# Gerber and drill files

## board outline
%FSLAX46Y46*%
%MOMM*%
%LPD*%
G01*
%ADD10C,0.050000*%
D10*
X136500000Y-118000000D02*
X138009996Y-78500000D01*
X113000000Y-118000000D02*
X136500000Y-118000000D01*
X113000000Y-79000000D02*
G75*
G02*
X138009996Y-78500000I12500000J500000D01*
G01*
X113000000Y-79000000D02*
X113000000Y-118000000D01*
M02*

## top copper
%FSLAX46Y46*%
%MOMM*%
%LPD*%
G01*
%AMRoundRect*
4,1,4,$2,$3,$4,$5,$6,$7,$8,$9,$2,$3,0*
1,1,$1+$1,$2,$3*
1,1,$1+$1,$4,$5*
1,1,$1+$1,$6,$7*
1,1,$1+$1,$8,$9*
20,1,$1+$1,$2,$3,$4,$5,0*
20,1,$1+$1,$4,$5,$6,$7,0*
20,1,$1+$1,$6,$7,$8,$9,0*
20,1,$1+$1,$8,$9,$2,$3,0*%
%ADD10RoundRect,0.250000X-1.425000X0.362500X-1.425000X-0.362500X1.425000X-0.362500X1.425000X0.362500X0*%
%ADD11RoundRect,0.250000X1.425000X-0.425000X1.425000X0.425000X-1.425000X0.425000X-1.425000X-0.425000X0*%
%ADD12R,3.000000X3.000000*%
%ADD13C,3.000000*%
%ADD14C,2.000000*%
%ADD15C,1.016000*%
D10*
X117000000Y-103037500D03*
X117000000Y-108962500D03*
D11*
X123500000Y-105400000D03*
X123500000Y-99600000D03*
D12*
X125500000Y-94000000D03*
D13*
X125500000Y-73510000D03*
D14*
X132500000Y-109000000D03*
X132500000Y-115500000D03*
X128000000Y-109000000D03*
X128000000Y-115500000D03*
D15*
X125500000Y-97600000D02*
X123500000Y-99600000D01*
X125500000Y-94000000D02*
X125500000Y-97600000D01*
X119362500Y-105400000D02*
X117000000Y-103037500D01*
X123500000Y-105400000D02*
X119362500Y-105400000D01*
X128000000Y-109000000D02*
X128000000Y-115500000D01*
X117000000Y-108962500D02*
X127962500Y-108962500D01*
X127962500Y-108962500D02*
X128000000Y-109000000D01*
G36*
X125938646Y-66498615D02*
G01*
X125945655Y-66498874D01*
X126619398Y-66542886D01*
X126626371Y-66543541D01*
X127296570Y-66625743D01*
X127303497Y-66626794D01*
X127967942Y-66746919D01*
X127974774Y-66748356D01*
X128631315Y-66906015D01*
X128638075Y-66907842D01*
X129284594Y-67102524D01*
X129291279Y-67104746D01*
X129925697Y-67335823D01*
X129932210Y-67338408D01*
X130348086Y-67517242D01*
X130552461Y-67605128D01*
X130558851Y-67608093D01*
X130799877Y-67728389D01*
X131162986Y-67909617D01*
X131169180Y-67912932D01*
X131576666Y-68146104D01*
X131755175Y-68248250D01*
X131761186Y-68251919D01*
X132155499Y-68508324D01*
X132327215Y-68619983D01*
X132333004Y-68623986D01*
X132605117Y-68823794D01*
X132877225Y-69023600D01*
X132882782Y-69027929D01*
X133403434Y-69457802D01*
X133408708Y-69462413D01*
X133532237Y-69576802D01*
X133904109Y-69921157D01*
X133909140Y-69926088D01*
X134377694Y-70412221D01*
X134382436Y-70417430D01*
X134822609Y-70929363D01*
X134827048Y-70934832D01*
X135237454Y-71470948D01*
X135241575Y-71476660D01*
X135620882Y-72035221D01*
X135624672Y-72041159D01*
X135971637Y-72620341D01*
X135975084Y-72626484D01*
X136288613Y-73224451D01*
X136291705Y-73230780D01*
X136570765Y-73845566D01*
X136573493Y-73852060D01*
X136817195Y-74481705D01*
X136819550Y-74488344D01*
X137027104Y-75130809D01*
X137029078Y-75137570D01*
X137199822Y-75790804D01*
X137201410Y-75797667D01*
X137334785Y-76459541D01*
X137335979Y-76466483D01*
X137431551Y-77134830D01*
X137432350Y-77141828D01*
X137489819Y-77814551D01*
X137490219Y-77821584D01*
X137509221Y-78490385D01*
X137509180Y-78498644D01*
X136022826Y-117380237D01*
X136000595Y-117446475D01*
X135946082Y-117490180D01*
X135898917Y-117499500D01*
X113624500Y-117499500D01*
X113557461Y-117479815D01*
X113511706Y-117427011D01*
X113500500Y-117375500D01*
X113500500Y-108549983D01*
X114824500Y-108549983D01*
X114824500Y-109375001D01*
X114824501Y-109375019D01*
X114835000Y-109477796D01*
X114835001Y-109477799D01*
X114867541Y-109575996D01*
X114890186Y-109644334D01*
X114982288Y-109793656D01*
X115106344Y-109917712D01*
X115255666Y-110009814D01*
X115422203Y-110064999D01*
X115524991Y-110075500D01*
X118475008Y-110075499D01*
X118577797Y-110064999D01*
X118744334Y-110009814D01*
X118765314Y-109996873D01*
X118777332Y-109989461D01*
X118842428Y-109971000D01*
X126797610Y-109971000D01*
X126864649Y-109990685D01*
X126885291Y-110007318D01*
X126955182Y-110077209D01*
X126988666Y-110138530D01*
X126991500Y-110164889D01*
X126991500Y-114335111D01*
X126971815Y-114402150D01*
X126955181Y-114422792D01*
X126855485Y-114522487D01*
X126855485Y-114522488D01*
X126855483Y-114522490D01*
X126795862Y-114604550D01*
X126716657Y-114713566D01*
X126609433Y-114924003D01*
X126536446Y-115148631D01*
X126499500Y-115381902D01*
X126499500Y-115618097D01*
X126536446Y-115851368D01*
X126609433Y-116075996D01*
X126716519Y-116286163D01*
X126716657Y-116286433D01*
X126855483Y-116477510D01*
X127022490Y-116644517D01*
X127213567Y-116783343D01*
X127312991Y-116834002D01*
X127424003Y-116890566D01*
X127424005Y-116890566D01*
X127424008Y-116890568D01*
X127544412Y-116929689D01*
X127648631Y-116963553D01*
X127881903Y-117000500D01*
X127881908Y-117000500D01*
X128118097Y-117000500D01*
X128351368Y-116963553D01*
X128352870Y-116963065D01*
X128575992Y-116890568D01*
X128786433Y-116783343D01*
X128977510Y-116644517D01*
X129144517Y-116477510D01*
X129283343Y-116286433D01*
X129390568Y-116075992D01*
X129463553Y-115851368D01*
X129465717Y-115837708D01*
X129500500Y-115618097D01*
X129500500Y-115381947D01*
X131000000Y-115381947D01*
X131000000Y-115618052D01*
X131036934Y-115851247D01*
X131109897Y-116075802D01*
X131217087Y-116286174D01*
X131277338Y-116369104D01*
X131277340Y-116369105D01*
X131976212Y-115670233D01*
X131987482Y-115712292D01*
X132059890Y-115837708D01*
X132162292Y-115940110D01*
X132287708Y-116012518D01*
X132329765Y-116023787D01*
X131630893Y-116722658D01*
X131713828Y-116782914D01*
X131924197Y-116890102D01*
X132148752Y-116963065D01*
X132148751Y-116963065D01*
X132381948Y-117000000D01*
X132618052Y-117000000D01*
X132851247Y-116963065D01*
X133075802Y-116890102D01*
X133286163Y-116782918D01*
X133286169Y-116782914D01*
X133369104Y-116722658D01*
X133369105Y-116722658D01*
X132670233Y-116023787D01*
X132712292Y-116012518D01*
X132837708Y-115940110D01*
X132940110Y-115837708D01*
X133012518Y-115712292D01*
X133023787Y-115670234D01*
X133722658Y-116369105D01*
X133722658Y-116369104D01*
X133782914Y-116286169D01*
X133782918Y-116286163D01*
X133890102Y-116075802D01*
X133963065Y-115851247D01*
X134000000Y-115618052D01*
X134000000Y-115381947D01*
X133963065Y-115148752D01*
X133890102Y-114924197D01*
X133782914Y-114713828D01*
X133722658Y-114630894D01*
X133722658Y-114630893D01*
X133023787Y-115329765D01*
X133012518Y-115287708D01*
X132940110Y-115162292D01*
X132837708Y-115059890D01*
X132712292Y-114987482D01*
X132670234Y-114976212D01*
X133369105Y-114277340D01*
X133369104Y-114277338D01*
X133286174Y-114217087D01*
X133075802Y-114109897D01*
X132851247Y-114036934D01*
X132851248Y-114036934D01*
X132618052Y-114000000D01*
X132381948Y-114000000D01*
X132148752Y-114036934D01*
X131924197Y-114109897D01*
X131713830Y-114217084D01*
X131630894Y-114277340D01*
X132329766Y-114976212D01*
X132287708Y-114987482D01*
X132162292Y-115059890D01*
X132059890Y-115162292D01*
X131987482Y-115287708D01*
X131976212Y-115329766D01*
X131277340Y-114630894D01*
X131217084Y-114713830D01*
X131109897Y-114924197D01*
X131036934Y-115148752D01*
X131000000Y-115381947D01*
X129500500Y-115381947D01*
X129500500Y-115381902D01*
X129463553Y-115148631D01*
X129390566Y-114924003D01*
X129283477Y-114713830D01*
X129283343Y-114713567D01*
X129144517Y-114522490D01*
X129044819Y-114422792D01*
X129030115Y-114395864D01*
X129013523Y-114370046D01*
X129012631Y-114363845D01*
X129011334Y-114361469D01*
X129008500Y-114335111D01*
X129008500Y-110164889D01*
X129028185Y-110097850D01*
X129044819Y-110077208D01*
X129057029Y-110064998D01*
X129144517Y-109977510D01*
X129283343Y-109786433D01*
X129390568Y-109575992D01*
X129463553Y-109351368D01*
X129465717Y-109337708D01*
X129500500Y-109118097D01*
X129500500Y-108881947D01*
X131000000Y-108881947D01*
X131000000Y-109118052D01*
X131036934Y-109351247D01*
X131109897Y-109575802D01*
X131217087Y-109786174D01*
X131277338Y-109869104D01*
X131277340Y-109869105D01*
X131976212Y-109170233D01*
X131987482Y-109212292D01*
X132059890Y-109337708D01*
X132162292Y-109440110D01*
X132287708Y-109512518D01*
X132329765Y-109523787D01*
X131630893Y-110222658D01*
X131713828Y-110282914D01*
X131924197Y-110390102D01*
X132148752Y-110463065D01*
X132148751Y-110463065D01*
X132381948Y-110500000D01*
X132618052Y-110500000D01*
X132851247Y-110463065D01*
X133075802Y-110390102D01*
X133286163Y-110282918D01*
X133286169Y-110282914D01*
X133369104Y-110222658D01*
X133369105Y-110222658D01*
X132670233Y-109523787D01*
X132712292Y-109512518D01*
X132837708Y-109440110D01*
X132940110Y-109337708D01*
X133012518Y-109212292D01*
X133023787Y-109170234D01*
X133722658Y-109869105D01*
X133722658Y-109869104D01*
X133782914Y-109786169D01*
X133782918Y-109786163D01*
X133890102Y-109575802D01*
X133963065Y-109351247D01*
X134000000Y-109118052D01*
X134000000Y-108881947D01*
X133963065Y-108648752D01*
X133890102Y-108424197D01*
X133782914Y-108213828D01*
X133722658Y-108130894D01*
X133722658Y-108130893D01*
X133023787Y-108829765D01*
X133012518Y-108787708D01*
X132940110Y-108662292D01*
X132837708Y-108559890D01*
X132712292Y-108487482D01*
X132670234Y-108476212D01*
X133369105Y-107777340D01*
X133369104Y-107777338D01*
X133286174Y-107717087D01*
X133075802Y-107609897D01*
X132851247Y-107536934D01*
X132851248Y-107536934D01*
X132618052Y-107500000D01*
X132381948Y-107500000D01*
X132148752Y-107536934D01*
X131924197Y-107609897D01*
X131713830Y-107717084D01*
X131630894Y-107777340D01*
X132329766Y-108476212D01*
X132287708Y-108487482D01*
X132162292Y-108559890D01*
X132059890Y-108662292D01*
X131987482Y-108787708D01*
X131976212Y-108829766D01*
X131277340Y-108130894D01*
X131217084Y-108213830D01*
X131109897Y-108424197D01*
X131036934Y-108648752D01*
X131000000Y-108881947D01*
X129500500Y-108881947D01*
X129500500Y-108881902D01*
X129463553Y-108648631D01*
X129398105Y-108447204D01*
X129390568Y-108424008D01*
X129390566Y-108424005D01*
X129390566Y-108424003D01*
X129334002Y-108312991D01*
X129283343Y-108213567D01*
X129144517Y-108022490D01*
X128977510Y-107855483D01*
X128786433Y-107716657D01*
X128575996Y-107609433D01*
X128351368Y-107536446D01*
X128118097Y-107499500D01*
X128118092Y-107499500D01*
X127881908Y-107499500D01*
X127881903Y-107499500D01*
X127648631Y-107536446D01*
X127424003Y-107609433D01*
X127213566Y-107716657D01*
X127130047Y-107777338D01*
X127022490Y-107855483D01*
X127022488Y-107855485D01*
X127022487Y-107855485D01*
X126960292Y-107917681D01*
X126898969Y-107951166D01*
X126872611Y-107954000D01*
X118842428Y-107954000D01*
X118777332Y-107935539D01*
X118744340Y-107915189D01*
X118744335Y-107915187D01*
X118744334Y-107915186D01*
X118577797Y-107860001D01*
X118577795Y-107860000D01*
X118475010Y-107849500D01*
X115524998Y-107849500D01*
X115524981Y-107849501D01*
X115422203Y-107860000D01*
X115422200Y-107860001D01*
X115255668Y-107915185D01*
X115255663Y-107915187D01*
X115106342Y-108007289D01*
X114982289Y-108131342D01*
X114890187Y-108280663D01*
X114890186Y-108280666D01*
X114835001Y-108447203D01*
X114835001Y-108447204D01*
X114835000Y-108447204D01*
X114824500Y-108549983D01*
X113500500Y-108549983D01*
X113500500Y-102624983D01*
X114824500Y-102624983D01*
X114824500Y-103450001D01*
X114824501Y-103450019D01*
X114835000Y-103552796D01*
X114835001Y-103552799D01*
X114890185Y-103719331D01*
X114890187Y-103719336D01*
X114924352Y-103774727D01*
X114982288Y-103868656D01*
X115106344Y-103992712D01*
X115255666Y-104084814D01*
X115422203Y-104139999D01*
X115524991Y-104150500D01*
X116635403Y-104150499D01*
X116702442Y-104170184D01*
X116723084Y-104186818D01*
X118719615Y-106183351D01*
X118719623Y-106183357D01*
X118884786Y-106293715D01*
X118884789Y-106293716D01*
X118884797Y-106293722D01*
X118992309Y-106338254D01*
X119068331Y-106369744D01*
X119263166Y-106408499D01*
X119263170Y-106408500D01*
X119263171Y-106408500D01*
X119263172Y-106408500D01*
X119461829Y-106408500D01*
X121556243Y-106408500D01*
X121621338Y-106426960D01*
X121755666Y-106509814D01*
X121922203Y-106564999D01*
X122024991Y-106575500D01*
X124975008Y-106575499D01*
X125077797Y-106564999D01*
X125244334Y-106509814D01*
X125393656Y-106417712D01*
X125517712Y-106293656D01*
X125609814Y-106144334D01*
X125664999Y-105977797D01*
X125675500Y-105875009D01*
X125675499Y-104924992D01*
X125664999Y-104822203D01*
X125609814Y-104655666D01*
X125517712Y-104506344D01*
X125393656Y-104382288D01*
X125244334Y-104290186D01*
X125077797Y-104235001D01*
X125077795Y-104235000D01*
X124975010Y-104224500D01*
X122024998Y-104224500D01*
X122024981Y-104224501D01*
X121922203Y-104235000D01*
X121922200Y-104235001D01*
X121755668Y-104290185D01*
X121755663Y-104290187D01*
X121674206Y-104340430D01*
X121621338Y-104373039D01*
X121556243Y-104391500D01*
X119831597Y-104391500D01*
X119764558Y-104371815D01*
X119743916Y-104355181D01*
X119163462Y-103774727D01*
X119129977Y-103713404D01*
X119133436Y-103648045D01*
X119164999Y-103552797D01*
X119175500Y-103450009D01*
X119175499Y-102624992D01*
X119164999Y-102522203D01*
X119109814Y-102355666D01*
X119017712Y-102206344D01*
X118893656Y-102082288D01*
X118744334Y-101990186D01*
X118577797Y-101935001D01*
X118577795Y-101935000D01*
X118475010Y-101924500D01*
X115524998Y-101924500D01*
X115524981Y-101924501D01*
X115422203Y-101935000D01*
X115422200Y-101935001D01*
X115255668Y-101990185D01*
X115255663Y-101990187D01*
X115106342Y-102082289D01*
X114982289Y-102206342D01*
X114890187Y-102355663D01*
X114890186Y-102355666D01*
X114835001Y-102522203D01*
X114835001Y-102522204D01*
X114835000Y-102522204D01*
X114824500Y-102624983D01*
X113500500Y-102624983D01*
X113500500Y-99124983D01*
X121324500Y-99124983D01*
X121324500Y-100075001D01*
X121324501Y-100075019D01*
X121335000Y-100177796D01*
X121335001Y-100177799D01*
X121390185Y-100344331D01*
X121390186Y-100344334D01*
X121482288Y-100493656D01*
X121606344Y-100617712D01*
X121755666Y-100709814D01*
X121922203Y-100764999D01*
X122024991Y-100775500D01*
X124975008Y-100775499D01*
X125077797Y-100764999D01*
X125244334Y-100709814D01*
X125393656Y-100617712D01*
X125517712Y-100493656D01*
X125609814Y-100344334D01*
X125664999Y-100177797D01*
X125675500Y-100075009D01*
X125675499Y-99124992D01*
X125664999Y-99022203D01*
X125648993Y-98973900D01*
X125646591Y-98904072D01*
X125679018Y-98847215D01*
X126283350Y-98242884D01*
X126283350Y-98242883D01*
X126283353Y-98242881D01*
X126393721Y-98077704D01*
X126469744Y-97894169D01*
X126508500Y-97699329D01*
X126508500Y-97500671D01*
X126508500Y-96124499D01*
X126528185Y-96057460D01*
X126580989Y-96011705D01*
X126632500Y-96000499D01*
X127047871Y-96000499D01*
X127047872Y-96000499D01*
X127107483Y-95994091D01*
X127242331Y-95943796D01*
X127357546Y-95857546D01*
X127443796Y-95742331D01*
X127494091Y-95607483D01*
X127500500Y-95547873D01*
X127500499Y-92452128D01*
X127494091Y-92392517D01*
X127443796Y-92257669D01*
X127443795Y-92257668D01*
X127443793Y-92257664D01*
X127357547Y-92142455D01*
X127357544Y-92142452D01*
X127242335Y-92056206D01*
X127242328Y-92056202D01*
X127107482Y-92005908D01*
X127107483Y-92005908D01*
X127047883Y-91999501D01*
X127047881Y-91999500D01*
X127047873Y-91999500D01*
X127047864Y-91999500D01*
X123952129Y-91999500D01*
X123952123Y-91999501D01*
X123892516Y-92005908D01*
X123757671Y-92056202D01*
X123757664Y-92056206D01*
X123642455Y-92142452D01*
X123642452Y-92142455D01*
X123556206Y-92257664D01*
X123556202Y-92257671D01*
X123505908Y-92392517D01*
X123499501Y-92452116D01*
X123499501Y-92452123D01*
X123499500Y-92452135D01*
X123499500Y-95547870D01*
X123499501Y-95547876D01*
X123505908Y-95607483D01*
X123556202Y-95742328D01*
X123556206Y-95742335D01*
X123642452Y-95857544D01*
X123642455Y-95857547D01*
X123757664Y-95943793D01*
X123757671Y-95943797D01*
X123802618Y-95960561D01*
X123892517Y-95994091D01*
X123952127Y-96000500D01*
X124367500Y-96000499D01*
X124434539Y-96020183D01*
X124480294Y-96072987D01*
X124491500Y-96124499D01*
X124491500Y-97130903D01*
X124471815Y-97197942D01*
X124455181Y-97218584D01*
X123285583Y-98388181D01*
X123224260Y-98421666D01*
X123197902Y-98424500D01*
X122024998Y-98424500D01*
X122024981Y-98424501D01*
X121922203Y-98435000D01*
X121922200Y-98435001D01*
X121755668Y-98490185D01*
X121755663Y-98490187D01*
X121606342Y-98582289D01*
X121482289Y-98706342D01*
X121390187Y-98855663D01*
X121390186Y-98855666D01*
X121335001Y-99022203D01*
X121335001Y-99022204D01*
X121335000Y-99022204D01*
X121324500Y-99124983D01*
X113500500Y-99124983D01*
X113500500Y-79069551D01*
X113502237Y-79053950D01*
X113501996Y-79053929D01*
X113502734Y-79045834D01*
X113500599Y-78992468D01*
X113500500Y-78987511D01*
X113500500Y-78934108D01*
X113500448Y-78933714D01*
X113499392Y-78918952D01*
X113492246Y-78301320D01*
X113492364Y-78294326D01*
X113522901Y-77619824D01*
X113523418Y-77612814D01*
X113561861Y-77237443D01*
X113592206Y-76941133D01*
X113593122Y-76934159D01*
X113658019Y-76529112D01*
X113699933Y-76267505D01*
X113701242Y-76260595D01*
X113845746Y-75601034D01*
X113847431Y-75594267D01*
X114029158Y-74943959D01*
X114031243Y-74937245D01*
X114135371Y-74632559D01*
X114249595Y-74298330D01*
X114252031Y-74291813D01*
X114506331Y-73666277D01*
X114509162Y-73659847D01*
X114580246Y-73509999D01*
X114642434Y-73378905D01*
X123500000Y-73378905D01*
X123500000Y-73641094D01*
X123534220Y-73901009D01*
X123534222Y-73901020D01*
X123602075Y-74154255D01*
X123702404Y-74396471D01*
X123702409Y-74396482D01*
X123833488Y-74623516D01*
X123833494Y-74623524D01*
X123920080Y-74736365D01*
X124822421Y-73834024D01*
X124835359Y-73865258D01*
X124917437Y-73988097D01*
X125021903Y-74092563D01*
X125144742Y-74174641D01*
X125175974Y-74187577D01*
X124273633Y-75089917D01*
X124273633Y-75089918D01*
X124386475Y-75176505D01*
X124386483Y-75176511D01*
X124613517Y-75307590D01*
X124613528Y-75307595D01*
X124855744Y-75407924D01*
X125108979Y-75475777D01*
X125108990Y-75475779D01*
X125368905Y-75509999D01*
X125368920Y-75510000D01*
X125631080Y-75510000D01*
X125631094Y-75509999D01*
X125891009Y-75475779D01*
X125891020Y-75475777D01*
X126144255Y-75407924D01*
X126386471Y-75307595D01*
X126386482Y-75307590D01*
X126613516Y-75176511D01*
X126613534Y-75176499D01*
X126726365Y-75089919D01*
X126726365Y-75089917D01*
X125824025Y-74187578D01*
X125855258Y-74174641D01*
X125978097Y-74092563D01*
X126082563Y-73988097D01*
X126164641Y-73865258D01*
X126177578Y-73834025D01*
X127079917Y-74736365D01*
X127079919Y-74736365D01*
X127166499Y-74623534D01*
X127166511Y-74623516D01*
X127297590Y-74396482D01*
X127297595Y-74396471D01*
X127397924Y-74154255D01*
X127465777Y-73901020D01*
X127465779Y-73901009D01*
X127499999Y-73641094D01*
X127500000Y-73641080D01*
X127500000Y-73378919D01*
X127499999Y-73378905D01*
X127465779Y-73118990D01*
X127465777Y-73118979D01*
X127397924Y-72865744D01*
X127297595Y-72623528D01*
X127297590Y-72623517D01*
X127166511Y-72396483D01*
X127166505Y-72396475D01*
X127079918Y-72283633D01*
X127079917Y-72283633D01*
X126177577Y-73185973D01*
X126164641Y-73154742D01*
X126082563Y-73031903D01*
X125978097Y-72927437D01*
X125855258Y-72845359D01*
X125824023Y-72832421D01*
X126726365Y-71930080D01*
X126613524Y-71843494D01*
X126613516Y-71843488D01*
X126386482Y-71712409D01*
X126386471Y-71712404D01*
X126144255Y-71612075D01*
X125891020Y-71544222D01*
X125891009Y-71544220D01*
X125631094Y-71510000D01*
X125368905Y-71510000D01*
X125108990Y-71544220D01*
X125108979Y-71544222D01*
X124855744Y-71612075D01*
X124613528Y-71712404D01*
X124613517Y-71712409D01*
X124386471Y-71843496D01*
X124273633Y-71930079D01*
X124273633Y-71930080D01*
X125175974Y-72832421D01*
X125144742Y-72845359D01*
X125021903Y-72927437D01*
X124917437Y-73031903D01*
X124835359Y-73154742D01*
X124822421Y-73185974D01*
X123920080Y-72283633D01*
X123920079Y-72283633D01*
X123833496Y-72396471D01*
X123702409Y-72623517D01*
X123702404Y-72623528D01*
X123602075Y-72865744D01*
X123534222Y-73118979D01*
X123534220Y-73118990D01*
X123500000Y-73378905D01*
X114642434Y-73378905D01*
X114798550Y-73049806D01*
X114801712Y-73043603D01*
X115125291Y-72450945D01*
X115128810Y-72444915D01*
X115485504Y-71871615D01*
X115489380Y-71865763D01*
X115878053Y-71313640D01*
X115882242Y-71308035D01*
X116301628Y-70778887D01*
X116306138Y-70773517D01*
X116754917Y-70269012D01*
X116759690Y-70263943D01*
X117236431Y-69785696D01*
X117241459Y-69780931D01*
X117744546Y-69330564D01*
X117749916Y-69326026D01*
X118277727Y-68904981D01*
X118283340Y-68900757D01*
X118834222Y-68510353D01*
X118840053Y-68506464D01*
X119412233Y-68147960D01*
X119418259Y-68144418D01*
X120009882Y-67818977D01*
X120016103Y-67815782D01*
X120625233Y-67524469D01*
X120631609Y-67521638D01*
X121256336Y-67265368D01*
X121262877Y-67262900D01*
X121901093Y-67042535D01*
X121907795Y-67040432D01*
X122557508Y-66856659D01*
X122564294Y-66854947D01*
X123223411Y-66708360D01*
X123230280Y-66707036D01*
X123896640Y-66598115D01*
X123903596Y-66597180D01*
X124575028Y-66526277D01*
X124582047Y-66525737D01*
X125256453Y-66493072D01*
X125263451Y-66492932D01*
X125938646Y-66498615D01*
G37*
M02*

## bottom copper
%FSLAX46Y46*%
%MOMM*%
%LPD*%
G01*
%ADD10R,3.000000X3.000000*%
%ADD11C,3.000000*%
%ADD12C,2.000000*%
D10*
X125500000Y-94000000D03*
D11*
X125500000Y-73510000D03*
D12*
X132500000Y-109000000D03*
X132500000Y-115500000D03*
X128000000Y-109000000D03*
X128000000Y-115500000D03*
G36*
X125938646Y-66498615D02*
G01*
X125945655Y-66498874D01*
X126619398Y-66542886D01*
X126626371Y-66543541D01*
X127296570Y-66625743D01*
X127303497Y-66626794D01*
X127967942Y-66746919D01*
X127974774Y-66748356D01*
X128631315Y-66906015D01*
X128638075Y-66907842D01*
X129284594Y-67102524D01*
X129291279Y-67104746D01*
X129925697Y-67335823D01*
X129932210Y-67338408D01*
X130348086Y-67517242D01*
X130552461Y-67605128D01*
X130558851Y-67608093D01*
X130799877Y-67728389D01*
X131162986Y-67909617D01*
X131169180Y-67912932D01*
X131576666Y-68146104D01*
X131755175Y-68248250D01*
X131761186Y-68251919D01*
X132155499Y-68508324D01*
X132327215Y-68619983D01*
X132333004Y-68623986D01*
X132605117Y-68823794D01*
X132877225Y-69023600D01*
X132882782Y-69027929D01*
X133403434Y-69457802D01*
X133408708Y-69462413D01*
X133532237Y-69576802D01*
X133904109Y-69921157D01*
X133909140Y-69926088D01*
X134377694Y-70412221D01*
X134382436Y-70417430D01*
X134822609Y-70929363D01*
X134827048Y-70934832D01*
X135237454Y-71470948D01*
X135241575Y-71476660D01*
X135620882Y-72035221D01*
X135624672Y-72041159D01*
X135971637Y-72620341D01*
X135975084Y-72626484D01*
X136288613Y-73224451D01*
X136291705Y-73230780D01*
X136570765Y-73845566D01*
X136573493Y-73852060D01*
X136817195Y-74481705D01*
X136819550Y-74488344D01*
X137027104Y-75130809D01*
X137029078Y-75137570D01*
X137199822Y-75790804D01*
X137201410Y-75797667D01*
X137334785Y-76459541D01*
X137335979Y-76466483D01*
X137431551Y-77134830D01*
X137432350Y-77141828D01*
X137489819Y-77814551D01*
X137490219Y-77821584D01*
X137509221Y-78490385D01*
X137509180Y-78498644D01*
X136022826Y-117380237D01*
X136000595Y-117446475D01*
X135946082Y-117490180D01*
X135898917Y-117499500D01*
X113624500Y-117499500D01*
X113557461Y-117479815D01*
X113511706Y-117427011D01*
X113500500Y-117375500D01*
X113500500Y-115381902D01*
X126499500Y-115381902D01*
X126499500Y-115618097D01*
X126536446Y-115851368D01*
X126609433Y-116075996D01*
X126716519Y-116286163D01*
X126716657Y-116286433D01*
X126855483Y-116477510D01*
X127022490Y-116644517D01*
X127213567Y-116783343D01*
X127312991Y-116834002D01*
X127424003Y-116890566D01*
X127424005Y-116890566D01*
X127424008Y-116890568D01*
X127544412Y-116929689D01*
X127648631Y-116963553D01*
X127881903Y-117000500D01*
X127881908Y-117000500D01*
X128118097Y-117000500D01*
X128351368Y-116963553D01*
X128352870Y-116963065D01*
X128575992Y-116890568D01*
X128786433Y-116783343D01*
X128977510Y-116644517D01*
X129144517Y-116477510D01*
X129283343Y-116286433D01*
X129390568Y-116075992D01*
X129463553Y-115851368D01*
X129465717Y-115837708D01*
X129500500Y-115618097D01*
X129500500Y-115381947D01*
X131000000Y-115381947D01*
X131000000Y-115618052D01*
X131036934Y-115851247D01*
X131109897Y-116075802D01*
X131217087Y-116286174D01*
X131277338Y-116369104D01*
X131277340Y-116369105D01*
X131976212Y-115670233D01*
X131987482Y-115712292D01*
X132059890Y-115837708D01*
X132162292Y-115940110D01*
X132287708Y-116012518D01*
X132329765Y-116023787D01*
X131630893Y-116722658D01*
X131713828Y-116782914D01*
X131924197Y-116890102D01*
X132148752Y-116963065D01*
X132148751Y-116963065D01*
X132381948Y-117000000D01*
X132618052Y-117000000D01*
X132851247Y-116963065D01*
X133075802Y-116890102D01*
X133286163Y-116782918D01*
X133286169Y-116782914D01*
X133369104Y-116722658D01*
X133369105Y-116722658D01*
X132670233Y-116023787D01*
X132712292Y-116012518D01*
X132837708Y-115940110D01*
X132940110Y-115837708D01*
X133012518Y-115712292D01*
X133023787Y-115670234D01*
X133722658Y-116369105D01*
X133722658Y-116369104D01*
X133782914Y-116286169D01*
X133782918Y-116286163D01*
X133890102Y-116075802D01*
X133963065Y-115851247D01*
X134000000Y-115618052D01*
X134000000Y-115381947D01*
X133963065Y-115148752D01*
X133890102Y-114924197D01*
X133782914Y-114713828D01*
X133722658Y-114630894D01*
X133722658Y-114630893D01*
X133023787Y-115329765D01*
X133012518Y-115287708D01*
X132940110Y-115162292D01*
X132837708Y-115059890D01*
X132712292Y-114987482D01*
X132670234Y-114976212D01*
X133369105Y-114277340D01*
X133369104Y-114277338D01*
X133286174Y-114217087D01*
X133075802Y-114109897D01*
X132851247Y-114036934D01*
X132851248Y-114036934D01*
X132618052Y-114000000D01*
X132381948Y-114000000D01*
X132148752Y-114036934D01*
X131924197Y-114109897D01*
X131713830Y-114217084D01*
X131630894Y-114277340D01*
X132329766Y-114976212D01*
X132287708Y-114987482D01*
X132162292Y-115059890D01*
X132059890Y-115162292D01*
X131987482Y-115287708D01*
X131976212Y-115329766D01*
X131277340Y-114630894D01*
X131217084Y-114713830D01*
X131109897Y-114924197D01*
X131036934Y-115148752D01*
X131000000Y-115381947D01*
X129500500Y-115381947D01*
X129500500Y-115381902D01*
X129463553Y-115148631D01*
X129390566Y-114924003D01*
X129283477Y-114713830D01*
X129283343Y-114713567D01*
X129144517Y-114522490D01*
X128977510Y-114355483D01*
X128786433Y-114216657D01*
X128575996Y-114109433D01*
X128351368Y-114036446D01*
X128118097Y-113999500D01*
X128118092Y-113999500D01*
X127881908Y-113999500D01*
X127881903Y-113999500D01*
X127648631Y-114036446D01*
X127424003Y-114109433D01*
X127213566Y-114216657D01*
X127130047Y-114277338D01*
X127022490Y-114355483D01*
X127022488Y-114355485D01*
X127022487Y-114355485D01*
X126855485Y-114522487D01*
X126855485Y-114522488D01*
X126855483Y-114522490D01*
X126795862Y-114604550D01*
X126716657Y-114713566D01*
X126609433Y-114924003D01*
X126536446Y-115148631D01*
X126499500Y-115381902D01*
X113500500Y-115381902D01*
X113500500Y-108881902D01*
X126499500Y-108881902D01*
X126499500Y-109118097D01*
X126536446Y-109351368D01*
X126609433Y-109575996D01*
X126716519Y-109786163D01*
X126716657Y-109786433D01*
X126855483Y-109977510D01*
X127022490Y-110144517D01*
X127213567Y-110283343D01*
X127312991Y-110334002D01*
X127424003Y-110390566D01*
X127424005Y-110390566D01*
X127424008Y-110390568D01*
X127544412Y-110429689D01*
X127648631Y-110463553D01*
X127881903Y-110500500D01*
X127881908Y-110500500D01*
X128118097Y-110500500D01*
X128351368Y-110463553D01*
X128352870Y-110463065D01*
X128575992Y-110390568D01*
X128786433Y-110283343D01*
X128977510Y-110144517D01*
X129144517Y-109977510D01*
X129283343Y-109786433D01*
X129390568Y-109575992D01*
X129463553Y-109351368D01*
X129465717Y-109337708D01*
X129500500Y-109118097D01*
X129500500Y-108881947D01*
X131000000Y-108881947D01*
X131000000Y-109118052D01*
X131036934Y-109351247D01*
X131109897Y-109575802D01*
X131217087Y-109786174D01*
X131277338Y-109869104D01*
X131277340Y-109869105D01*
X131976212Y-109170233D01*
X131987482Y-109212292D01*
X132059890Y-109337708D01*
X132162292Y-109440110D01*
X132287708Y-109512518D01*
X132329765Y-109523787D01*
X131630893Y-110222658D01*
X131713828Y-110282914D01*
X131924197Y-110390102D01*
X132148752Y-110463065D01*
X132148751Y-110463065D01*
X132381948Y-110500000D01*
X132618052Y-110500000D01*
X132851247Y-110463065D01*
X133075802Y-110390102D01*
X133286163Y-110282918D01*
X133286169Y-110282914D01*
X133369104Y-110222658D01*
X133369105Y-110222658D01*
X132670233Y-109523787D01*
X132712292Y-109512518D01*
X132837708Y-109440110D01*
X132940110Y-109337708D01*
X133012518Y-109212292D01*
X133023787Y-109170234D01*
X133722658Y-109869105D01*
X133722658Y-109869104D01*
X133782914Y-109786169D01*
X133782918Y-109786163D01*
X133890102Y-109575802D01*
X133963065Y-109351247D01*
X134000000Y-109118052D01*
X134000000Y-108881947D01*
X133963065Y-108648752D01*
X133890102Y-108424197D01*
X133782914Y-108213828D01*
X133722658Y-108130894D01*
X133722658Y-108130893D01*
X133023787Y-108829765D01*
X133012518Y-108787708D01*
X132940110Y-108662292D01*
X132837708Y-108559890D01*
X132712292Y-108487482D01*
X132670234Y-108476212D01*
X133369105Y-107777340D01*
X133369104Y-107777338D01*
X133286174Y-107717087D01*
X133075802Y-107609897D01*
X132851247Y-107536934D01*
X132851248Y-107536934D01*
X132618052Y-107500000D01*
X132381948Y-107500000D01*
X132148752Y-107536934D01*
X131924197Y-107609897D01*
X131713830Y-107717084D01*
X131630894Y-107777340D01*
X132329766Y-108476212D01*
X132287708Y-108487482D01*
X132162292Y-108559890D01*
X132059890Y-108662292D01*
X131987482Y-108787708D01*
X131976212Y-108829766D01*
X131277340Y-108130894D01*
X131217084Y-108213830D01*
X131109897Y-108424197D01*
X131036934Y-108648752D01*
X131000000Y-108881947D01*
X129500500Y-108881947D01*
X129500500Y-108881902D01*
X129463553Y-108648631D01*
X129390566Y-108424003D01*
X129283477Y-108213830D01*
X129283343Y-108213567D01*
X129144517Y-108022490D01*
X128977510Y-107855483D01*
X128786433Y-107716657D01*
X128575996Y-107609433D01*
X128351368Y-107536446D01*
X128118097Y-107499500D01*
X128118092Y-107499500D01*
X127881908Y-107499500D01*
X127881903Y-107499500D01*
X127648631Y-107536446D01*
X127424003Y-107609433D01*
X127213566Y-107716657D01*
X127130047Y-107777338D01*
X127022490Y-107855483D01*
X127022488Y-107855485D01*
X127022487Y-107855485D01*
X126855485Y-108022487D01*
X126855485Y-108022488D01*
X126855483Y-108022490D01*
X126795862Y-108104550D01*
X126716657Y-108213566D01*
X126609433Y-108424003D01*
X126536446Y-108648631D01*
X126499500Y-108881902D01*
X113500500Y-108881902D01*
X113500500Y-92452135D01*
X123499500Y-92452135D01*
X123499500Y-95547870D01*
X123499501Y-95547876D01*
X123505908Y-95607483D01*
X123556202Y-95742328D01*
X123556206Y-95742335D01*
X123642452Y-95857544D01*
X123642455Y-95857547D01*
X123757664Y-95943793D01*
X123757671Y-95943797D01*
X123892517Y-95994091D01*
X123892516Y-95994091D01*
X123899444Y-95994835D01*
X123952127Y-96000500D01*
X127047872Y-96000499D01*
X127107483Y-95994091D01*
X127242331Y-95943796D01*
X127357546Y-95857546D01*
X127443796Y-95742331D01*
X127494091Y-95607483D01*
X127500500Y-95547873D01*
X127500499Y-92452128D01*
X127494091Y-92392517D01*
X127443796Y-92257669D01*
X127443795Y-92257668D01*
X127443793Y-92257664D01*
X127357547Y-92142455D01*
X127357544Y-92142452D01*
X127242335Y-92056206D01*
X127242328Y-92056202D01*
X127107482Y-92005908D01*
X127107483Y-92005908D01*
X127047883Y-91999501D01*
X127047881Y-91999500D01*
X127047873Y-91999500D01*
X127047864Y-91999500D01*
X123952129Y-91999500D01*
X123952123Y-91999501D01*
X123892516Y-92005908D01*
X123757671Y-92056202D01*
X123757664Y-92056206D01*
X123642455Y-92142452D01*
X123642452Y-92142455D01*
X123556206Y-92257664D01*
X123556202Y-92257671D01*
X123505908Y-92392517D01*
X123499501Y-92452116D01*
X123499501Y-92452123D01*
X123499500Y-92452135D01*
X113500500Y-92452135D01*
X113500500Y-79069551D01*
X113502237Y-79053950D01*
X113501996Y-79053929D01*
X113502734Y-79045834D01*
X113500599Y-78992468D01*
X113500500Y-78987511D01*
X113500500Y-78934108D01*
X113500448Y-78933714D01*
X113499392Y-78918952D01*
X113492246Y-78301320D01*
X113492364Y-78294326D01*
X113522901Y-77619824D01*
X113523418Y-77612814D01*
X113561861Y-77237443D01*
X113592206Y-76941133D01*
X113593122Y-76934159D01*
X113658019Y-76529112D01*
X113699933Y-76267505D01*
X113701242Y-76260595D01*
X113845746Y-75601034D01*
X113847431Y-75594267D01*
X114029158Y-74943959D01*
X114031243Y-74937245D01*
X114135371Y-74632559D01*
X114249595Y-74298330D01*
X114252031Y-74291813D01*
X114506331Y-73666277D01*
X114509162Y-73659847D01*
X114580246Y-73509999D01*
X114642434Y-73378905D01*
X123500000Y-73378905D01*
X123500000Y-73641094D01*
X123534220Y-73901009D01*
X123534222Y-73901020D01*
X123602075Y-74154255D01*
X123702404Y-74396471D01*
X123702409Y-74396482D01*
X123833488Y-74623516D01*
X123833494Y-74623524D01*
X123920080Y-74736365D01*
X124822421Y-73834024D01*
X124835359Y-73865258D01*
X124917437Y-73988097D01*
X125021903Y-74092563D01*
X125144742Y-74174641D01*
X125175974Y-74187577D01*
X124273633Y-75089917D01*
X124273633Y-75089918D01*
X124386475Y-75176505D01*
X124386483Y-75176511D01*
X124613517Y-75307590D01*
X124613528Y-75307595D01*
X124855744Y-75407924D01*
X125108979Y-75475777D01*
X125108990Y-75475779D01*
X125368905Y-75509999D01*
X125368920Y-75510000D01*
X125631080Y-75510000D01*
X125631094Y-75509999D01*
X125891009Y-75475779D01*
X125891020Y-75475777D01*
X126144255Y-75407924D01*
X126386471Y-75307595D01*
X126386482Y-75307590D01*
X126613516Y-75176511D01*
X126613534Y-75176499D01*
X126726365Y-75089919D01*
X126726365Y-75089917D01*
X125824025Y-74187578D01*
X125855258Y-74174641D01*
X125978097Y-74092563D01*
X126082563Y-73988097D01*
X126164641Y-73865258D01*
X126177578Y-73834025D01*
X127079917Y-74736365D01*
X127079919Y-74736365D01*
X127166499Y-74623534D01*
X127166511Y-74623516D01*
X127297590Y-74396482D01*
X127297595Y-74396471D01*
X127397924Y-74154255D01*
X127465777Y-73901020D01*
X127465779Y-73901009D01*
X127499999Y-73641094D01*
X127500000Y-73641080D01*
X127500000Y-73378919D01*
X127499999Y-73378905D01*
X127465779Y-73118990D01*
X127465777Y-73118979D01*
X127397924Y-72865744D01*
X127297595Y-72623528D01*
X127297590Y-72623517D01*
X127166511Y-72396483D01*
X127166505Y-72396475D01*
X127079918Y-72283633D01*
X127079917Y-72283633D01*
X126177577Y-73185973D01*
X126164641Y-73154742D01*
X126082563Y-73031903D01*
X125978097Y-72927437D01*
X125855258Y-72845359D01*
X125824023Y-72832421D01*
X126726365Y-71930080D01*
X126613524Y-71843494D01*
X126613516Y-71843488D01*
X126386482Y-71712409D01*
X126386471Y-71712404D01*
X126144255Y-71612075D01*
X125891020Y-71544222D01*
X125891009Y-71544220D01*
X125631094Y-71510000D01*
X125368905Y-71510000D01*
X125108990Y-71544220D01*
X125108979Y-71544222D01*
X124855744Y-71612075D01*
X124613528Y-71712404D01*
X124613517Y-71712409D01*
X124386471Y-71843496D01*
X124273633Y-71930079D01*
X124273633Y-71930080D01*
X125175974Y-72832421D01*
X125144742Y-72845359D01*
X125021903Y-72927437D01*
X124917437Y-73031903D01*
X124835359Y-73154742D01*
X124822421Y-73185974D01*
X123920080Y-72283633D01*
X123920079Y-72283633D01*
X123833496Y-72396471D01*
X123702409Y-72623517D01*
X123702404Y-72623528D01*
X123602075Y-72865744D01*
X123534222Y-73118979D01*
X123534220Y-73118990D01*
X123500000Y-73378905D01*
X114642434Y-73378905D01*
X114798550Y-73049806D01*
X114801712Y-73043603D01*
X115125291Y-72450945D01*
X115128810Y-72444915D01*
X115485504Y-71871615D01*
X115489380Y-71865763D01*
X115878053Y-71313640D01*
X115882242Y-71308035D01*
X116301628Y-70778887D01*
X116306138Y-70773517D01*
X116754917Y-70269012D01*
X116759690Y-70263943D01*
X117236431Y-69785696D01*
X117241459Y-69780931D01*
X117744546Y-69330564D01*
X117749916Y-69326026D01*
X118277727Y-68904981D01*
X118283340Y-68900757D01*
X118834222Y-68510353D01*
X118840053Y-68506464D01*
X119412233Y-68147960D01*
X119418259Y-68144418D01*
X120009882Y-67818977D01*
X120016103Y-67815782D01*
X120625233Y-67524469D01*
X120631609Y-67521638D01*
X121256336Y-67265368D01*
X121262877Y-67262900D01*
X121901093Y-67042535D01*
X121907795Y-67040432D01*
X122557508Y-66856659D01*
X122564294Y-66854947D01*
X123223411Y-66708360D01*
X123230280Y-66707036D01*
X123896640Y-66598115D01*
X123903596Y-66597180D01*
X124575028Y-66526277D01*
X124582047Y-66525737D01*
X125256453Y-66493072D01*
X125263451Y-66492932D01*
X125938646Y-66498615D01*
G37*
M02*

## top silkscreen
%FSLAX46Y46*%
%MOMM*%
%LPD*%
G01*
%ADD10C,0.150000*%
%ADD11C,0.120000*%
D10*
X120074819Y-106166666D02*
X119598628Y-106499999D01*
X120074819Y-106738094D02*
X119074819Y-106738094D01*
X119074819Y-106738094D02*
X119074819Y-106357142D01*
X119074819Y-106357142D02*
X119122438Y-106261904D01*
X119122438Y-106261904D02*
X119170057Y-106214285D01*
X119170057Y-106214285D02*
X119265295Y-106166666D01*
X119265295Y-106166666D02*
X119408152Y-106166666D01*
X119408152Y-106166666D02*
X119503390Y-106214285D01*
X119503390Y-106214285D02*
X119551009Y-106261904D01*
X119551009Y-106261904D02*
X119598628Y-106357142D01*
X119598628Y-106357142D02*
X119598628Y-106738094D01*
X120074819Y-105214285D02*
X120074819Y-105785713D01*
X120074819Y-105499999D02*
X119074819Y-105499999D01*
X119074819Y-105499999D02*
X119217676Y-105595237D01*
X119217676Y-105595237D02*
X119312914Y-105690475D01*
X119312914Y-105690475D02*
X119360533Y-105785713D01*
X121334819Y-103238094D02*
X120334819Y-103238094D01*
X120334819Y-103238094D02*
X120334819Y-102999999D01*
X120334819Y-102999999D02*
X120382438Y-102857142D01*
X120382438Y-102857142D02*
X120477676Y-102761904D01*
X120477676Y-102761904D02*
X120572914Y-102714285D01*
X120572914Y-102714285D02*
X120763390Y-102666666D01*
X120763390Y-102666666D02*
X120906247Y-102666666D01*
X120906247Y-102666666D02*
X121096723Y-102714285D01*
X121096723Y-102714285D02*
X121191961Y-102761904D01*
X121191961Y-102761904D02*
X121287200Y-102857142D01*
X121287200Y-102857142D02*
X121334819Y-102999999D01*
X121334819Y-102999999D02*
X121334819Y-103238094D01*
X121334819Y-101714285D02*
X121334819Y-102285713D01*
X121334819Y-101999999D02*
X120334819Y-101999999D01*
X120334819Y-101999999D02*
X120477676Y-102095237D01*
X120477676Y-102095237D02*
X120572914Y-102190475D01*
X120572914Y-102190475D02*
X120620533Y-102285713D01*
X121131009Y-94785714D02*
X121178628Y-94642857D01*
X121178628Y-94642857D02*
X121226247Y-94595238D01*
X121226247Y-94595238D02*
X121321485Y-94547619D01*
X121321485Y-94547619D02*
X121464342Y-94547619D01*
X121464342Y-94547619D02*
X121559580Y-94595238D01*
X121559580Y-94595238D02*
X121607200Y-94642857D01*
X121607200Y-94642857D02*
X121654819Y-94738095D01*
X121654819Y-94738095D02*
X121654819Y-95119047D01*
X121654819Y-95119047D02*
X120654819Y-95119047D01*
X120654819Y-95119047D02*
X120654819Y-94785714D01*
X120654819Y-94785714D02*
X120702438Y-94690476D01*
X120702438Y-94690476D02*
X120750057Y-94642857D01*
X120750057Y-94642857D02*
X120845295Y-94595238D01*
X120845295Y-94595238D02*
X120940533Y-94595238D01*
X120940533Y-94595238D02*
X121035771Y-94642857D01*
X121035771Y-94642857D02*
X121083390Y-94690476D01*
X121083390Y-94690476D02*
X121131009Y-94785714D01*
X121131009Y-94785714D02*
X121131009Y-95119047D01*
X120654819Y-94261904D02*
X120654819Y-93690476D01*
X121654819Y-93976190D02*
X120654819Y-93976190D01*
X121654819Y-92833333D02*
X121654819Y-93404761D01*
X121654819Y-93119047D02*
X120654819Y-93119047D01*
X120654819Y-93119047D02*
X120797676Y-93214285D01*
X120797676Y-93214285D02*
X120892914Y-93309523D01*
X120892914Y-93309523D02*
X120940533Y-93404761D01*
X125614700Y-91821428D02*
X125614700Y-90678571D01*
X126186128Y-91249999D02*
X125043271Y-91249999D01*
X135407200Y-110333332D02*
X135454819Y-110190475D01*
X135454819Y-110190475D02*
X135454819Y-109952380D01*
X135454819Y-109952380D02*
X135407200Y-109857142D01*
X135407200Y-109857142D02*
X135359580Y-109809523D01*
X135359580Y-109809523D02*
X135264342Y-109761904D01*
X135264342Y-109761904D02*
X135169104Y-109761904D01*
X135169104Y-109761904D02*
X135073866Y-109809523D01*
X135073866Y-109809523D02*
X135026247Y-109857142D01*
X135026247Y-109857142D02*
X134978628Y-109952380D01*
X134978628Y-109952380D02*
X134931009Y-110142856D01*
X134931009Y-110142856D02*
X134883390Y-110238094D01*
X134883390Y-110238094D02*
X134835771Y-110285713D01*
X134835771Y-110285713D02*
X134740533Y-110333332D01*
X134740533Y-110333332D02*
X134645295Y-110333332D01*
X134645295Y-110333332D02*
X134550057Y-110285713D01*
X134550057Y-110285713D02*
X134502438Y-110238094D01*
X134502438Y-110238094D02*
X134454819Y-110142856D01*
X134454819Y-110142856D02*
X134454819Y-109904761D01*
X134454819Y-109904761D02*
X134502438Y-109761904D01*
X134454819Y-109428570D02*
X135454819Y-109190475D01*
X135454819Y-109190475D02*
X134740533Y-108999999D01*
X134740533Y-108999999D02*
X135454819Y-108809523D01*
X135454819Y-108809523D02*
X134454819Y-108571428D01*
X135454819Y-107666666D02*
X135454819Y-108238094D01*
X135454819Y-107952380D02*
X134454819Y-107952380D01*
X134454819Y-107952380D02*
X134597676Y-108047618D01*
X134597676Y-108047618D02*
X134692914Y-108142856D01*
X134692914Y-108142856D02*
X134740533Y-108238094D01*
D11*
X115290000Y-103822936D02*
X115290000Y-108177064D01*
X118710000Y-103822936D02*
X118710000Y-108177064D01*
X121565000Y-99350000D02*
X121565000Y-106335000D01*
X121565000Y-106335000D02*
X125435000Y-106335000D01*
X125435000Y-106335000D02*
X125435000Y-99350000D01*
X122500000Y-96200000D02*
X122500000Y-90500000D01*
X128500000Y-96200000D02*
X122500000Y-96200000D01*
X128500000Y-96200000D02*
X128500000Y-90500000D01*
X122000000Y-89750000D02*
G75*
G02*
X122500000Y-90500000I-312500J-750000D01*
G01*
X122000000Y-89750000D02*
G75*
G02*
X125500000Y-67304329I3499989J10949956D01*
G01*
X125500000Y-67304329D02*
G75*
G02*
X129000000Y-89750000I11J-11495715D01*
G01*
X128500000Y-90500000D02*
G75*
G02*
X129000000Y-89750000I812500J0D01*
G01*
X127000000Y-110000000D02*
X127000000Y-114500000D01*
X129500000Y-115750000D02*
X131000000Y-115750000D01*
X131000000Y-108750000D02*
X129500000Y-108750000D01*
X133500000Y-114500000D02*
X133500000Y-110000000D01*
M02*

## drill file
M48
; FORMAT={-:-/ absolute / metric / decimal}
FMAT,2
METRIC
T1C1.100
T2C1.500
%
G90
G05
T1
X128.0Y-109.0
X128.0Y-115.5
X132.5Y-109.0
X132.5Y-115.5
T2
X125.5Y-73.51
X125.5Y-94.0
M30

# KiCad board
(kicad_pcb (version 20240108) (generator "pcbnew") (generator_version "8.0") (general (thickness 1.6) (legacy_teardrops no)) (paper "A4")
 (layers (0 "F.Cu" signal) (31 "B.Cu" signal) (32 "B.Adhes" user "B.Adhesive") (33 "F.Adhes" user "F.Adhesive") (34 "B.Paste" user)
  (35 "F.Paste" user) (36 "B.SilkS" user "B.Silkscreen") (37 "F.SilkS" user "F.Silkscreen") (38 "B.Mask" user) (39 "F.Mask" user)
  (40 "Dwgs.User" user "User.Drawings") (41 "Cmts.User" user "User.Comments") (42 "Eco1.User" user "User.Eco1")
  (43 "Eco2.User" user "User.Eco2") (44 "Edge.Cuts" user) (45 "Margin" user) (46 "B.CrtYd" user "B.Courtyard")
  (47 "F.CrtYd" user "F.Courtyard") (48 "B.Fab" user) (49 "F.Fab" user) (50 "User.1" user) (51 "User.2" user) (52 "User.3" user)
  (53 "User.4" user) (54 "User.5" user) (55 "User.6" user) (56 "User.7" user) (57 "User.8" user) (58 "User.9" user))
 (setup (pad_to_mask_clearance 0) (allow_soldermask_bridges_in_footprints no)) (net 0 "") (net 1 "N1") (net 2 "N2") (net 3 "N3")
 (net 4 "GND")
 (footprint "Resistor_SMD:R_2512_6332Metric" (layer "F.Cu") (at 117 106 -90)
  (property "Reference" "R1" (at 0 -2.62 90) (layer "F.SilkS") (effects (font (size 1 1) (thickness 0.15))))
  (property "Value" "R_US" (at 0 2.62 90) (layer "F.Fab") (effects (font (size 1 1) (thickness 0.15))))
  (fp_line (start -2.177064 1.71) (end 2.177064 1.71) (stroke (width 0.12) (type solid)) (layer "F.SilkS"))
  (fp_line (start -2.177064 -1.71) (end 2.177064 -1.71) (stroke (width 0.12) (type solid)) (layer "F.SilkS"))
  (pad "1" smd roundrect (at -2.9625 0 270) (size 1.225 3.35) (layers "F.Cu" "F.Paste" "F.Mask") (roundrect_rratio 0.204082) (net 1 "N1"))
  (pad "2" smd roundrect (at 2.9625 0 270) (size 1.225 3.35) (layers "F.Cu" "F.Paste" "F.Mask") (roundrect_rratio 0.204082) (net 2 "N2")))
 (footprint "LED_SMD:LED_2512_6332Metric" (layer "F.Cu") (at 123.5 102.5 90)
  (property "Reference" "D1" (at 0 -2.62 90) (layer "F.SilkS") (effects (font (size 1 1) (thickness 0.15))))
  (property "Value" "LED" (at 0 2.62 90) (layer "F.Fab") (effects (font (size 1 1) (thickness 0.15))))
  (fp_line (start 3.15 -1.935) (end -3.835 -1.935) (stroke (width 0.12) (type solid)) (layer "F.SilkS"))
  (fp_line (start -3.835 -1.935) (end -3.835 1.935) (stroke (width 0.12) (type solid)) (layer "F.SilkS"))
  (fp_line (start -3.835 1.935) (end 3.15 1.935) (stroke (width 0.12) (type solid)) (layer "F.SilkS"))
  (pad "1" smd roundrect (at -2.9 0 90) (size 1.35 3.35) (layers "F.Cu" "F.Paste" "F.Mask") (roundrect_rratio 0.185185) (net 1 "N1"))
  (pad "2" smd roundrect (at 2.9 0 90) (size 1.35 3.35) (layers "F.Cu" "F.Paste" "F.Mask") (roundrect_rratio 0.185185) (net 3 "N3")))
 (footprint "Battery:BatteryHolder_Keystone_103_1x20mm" (layer "F.Cu") (at 125.5 94 90)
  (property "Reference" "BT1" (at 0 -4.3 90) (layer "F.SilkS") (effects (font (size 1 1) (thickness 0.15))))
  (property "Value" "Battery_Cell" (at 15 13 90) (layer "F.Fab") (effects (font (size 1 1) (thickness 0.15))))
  (fp_line (start -2.2 -3) (end 3.5 -3) (stroke (width 0.12) (type solid)) (layer "F.SilkS"))
  (fp_line (start -2.2 3) (end -2.2 -3) (stroke (width 0.12) (type solid)) (layer "F.SilkS"))
  (fp_line (start -2.2 3) (end 3.5 3) (stroke (width 0.12) (type solid)) (layer "F.SilkS"))
  (fp_arc (start 4.25 -3.5) (mid 3.950694 -3.136459) (end 3.5 -3) (stroke (width 0.12) (type solid)) (layer "F.SilkS"))
  (fp_arc (start 4.25 -3.5) (mid 16.971103 -11.358466) (end 26.695671 0) (stroke (width 0.12) (type solid)) (layer "F.SilkS"))
  (fp_arc (start 26.695671 0) (mid 16.971103 11.358466) (end 4.25 3.5) (stroke (width 0.12) (type solid)) (layer "F.SilkS"))
  (fp_arc (start 3.5 3) (mid 3.950694 3.136459) (end 4.25 3.5) (stroke (width 0.12) (type solid)) (layer "F.SilkS"))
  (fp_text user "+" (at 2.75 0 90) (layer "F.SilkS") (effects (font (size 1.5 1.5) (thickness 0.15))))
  (pad "1" thru_hole rect (at 0 0 90) (size 3 3) (drill 1.5) (layers "*.Cu" "*.Mask") (remove_unused_layers no) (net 3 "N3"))
  (pad "2" thru_hole circle (at 20.49 0 90) (size 3 3) (drill 1.5) (layers "*.Cu" "*.Mask") (remove_unused_layers no) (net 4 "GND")))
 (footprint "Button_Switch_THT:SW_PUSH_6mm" (layer "F.Cu") (at 132.5 109 -90)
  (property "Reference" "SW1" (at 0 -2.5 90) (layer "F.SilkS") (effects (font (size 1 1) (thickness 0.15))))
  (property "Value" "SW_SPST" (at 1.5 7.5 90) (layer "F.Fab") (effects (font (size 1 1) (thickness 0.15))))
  (fp_line (start 1 5.5) (end 5.5 5.5) (stroke (width 0.12) (type solid)) (layer "F.SilkS"))
  (fp_line (start 6.75 3) (end 6.75 1.5) (stroke (width 0.12) (type solid)) (layer "F.SilkS"))
  (fp_line (start -0.25 1.5) (end -0.25 3) (stroke (width 0.12) (type solid)) (layer "F.SilkS"))
  (fp_line (start 5.5 -1) (end 1 -1) (stroke (width 0.12) (type solid)) (layer "F.SilkS"))
  (pad "1" thru_hole circle (at 0 0) (size 2 2) (drill 1.1) (layers "*.Cu" "*.Mask") (remove_unused_layers no) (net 4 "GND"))
  (pad "1" thru_hole circle (at 6.5 0) (size 2 2) (drill 1.1) (layers "*.Cu" "*.Mask") (remove_unused_layers no) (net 4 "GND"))
  (pad "2" thru_hole circle (at 0 4.5) (size 2 2) (drill 1.1) (layers "*.Cu" "*.Mask") (remove_unused_layers no) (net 2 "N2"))
  (pad "2" thru_hole circle (at 6.5 4.5) (size 2 2) (drill 1.1) (layers "*.Cu" "*.Mask") (remove_unused_layers no) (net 2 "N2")))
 (gr_line (start 136.5 118) (end 138.009996 78.5) (stroke (width 0.05) (type default)) (layer "Edge.Cuts"))
 (gr_line (start 113 118) (end 136.5 118) (stroke (width 0.05) (type default)) (layer "Edge.Cuts"))
 (gr_arc (start 113 79) (mid 125.24995 65.992503) (end 138.009996 78.5) (stroke (width 0.05) (type default)) (layer "Edge.Cuts"))
 (gr_line (start 113 79) (end 113 118) (stroke (width 0.05) (type default)) (layer "Edge.Cuts"))
 (segment (start 125.5 97.6) (end 123.5 99.6) (width 1.016) (layer "F.Cu") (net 3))
 (segment (start 125.5 94) (end 125.5 97.6) (width 1.016) (layer "F.Cu") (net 3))
 (segment (start 119.3625 105.4) (end 117 103.0375) (width 1.016) (layer "F.Cu") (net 1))
 (segment (start 123.5 105.4) (end 119.3625 105.4) (width 1.016) (layer "F.Cu") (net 1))
 (segment (start 128 109) (end 128 115.5) (width 1.016) (layer "F.Cu") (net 2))
 (segment (start 117 108.9625) (end 127.9625 108.9625) (width 1.016) (layer "F.Cu") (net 2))
 (segment (start 127.9625 108.9625) (end 128 109) (width 1.016) (layer "F.Cu") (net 2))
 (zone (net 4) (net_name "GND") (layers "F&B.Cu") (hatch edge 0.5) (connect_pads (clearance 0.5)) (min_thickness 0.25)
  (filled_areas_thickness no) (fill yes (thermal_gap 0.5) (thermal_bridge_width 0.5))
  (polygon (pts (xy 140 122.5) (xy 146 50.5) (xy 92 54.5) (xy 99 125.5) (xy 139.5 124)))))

